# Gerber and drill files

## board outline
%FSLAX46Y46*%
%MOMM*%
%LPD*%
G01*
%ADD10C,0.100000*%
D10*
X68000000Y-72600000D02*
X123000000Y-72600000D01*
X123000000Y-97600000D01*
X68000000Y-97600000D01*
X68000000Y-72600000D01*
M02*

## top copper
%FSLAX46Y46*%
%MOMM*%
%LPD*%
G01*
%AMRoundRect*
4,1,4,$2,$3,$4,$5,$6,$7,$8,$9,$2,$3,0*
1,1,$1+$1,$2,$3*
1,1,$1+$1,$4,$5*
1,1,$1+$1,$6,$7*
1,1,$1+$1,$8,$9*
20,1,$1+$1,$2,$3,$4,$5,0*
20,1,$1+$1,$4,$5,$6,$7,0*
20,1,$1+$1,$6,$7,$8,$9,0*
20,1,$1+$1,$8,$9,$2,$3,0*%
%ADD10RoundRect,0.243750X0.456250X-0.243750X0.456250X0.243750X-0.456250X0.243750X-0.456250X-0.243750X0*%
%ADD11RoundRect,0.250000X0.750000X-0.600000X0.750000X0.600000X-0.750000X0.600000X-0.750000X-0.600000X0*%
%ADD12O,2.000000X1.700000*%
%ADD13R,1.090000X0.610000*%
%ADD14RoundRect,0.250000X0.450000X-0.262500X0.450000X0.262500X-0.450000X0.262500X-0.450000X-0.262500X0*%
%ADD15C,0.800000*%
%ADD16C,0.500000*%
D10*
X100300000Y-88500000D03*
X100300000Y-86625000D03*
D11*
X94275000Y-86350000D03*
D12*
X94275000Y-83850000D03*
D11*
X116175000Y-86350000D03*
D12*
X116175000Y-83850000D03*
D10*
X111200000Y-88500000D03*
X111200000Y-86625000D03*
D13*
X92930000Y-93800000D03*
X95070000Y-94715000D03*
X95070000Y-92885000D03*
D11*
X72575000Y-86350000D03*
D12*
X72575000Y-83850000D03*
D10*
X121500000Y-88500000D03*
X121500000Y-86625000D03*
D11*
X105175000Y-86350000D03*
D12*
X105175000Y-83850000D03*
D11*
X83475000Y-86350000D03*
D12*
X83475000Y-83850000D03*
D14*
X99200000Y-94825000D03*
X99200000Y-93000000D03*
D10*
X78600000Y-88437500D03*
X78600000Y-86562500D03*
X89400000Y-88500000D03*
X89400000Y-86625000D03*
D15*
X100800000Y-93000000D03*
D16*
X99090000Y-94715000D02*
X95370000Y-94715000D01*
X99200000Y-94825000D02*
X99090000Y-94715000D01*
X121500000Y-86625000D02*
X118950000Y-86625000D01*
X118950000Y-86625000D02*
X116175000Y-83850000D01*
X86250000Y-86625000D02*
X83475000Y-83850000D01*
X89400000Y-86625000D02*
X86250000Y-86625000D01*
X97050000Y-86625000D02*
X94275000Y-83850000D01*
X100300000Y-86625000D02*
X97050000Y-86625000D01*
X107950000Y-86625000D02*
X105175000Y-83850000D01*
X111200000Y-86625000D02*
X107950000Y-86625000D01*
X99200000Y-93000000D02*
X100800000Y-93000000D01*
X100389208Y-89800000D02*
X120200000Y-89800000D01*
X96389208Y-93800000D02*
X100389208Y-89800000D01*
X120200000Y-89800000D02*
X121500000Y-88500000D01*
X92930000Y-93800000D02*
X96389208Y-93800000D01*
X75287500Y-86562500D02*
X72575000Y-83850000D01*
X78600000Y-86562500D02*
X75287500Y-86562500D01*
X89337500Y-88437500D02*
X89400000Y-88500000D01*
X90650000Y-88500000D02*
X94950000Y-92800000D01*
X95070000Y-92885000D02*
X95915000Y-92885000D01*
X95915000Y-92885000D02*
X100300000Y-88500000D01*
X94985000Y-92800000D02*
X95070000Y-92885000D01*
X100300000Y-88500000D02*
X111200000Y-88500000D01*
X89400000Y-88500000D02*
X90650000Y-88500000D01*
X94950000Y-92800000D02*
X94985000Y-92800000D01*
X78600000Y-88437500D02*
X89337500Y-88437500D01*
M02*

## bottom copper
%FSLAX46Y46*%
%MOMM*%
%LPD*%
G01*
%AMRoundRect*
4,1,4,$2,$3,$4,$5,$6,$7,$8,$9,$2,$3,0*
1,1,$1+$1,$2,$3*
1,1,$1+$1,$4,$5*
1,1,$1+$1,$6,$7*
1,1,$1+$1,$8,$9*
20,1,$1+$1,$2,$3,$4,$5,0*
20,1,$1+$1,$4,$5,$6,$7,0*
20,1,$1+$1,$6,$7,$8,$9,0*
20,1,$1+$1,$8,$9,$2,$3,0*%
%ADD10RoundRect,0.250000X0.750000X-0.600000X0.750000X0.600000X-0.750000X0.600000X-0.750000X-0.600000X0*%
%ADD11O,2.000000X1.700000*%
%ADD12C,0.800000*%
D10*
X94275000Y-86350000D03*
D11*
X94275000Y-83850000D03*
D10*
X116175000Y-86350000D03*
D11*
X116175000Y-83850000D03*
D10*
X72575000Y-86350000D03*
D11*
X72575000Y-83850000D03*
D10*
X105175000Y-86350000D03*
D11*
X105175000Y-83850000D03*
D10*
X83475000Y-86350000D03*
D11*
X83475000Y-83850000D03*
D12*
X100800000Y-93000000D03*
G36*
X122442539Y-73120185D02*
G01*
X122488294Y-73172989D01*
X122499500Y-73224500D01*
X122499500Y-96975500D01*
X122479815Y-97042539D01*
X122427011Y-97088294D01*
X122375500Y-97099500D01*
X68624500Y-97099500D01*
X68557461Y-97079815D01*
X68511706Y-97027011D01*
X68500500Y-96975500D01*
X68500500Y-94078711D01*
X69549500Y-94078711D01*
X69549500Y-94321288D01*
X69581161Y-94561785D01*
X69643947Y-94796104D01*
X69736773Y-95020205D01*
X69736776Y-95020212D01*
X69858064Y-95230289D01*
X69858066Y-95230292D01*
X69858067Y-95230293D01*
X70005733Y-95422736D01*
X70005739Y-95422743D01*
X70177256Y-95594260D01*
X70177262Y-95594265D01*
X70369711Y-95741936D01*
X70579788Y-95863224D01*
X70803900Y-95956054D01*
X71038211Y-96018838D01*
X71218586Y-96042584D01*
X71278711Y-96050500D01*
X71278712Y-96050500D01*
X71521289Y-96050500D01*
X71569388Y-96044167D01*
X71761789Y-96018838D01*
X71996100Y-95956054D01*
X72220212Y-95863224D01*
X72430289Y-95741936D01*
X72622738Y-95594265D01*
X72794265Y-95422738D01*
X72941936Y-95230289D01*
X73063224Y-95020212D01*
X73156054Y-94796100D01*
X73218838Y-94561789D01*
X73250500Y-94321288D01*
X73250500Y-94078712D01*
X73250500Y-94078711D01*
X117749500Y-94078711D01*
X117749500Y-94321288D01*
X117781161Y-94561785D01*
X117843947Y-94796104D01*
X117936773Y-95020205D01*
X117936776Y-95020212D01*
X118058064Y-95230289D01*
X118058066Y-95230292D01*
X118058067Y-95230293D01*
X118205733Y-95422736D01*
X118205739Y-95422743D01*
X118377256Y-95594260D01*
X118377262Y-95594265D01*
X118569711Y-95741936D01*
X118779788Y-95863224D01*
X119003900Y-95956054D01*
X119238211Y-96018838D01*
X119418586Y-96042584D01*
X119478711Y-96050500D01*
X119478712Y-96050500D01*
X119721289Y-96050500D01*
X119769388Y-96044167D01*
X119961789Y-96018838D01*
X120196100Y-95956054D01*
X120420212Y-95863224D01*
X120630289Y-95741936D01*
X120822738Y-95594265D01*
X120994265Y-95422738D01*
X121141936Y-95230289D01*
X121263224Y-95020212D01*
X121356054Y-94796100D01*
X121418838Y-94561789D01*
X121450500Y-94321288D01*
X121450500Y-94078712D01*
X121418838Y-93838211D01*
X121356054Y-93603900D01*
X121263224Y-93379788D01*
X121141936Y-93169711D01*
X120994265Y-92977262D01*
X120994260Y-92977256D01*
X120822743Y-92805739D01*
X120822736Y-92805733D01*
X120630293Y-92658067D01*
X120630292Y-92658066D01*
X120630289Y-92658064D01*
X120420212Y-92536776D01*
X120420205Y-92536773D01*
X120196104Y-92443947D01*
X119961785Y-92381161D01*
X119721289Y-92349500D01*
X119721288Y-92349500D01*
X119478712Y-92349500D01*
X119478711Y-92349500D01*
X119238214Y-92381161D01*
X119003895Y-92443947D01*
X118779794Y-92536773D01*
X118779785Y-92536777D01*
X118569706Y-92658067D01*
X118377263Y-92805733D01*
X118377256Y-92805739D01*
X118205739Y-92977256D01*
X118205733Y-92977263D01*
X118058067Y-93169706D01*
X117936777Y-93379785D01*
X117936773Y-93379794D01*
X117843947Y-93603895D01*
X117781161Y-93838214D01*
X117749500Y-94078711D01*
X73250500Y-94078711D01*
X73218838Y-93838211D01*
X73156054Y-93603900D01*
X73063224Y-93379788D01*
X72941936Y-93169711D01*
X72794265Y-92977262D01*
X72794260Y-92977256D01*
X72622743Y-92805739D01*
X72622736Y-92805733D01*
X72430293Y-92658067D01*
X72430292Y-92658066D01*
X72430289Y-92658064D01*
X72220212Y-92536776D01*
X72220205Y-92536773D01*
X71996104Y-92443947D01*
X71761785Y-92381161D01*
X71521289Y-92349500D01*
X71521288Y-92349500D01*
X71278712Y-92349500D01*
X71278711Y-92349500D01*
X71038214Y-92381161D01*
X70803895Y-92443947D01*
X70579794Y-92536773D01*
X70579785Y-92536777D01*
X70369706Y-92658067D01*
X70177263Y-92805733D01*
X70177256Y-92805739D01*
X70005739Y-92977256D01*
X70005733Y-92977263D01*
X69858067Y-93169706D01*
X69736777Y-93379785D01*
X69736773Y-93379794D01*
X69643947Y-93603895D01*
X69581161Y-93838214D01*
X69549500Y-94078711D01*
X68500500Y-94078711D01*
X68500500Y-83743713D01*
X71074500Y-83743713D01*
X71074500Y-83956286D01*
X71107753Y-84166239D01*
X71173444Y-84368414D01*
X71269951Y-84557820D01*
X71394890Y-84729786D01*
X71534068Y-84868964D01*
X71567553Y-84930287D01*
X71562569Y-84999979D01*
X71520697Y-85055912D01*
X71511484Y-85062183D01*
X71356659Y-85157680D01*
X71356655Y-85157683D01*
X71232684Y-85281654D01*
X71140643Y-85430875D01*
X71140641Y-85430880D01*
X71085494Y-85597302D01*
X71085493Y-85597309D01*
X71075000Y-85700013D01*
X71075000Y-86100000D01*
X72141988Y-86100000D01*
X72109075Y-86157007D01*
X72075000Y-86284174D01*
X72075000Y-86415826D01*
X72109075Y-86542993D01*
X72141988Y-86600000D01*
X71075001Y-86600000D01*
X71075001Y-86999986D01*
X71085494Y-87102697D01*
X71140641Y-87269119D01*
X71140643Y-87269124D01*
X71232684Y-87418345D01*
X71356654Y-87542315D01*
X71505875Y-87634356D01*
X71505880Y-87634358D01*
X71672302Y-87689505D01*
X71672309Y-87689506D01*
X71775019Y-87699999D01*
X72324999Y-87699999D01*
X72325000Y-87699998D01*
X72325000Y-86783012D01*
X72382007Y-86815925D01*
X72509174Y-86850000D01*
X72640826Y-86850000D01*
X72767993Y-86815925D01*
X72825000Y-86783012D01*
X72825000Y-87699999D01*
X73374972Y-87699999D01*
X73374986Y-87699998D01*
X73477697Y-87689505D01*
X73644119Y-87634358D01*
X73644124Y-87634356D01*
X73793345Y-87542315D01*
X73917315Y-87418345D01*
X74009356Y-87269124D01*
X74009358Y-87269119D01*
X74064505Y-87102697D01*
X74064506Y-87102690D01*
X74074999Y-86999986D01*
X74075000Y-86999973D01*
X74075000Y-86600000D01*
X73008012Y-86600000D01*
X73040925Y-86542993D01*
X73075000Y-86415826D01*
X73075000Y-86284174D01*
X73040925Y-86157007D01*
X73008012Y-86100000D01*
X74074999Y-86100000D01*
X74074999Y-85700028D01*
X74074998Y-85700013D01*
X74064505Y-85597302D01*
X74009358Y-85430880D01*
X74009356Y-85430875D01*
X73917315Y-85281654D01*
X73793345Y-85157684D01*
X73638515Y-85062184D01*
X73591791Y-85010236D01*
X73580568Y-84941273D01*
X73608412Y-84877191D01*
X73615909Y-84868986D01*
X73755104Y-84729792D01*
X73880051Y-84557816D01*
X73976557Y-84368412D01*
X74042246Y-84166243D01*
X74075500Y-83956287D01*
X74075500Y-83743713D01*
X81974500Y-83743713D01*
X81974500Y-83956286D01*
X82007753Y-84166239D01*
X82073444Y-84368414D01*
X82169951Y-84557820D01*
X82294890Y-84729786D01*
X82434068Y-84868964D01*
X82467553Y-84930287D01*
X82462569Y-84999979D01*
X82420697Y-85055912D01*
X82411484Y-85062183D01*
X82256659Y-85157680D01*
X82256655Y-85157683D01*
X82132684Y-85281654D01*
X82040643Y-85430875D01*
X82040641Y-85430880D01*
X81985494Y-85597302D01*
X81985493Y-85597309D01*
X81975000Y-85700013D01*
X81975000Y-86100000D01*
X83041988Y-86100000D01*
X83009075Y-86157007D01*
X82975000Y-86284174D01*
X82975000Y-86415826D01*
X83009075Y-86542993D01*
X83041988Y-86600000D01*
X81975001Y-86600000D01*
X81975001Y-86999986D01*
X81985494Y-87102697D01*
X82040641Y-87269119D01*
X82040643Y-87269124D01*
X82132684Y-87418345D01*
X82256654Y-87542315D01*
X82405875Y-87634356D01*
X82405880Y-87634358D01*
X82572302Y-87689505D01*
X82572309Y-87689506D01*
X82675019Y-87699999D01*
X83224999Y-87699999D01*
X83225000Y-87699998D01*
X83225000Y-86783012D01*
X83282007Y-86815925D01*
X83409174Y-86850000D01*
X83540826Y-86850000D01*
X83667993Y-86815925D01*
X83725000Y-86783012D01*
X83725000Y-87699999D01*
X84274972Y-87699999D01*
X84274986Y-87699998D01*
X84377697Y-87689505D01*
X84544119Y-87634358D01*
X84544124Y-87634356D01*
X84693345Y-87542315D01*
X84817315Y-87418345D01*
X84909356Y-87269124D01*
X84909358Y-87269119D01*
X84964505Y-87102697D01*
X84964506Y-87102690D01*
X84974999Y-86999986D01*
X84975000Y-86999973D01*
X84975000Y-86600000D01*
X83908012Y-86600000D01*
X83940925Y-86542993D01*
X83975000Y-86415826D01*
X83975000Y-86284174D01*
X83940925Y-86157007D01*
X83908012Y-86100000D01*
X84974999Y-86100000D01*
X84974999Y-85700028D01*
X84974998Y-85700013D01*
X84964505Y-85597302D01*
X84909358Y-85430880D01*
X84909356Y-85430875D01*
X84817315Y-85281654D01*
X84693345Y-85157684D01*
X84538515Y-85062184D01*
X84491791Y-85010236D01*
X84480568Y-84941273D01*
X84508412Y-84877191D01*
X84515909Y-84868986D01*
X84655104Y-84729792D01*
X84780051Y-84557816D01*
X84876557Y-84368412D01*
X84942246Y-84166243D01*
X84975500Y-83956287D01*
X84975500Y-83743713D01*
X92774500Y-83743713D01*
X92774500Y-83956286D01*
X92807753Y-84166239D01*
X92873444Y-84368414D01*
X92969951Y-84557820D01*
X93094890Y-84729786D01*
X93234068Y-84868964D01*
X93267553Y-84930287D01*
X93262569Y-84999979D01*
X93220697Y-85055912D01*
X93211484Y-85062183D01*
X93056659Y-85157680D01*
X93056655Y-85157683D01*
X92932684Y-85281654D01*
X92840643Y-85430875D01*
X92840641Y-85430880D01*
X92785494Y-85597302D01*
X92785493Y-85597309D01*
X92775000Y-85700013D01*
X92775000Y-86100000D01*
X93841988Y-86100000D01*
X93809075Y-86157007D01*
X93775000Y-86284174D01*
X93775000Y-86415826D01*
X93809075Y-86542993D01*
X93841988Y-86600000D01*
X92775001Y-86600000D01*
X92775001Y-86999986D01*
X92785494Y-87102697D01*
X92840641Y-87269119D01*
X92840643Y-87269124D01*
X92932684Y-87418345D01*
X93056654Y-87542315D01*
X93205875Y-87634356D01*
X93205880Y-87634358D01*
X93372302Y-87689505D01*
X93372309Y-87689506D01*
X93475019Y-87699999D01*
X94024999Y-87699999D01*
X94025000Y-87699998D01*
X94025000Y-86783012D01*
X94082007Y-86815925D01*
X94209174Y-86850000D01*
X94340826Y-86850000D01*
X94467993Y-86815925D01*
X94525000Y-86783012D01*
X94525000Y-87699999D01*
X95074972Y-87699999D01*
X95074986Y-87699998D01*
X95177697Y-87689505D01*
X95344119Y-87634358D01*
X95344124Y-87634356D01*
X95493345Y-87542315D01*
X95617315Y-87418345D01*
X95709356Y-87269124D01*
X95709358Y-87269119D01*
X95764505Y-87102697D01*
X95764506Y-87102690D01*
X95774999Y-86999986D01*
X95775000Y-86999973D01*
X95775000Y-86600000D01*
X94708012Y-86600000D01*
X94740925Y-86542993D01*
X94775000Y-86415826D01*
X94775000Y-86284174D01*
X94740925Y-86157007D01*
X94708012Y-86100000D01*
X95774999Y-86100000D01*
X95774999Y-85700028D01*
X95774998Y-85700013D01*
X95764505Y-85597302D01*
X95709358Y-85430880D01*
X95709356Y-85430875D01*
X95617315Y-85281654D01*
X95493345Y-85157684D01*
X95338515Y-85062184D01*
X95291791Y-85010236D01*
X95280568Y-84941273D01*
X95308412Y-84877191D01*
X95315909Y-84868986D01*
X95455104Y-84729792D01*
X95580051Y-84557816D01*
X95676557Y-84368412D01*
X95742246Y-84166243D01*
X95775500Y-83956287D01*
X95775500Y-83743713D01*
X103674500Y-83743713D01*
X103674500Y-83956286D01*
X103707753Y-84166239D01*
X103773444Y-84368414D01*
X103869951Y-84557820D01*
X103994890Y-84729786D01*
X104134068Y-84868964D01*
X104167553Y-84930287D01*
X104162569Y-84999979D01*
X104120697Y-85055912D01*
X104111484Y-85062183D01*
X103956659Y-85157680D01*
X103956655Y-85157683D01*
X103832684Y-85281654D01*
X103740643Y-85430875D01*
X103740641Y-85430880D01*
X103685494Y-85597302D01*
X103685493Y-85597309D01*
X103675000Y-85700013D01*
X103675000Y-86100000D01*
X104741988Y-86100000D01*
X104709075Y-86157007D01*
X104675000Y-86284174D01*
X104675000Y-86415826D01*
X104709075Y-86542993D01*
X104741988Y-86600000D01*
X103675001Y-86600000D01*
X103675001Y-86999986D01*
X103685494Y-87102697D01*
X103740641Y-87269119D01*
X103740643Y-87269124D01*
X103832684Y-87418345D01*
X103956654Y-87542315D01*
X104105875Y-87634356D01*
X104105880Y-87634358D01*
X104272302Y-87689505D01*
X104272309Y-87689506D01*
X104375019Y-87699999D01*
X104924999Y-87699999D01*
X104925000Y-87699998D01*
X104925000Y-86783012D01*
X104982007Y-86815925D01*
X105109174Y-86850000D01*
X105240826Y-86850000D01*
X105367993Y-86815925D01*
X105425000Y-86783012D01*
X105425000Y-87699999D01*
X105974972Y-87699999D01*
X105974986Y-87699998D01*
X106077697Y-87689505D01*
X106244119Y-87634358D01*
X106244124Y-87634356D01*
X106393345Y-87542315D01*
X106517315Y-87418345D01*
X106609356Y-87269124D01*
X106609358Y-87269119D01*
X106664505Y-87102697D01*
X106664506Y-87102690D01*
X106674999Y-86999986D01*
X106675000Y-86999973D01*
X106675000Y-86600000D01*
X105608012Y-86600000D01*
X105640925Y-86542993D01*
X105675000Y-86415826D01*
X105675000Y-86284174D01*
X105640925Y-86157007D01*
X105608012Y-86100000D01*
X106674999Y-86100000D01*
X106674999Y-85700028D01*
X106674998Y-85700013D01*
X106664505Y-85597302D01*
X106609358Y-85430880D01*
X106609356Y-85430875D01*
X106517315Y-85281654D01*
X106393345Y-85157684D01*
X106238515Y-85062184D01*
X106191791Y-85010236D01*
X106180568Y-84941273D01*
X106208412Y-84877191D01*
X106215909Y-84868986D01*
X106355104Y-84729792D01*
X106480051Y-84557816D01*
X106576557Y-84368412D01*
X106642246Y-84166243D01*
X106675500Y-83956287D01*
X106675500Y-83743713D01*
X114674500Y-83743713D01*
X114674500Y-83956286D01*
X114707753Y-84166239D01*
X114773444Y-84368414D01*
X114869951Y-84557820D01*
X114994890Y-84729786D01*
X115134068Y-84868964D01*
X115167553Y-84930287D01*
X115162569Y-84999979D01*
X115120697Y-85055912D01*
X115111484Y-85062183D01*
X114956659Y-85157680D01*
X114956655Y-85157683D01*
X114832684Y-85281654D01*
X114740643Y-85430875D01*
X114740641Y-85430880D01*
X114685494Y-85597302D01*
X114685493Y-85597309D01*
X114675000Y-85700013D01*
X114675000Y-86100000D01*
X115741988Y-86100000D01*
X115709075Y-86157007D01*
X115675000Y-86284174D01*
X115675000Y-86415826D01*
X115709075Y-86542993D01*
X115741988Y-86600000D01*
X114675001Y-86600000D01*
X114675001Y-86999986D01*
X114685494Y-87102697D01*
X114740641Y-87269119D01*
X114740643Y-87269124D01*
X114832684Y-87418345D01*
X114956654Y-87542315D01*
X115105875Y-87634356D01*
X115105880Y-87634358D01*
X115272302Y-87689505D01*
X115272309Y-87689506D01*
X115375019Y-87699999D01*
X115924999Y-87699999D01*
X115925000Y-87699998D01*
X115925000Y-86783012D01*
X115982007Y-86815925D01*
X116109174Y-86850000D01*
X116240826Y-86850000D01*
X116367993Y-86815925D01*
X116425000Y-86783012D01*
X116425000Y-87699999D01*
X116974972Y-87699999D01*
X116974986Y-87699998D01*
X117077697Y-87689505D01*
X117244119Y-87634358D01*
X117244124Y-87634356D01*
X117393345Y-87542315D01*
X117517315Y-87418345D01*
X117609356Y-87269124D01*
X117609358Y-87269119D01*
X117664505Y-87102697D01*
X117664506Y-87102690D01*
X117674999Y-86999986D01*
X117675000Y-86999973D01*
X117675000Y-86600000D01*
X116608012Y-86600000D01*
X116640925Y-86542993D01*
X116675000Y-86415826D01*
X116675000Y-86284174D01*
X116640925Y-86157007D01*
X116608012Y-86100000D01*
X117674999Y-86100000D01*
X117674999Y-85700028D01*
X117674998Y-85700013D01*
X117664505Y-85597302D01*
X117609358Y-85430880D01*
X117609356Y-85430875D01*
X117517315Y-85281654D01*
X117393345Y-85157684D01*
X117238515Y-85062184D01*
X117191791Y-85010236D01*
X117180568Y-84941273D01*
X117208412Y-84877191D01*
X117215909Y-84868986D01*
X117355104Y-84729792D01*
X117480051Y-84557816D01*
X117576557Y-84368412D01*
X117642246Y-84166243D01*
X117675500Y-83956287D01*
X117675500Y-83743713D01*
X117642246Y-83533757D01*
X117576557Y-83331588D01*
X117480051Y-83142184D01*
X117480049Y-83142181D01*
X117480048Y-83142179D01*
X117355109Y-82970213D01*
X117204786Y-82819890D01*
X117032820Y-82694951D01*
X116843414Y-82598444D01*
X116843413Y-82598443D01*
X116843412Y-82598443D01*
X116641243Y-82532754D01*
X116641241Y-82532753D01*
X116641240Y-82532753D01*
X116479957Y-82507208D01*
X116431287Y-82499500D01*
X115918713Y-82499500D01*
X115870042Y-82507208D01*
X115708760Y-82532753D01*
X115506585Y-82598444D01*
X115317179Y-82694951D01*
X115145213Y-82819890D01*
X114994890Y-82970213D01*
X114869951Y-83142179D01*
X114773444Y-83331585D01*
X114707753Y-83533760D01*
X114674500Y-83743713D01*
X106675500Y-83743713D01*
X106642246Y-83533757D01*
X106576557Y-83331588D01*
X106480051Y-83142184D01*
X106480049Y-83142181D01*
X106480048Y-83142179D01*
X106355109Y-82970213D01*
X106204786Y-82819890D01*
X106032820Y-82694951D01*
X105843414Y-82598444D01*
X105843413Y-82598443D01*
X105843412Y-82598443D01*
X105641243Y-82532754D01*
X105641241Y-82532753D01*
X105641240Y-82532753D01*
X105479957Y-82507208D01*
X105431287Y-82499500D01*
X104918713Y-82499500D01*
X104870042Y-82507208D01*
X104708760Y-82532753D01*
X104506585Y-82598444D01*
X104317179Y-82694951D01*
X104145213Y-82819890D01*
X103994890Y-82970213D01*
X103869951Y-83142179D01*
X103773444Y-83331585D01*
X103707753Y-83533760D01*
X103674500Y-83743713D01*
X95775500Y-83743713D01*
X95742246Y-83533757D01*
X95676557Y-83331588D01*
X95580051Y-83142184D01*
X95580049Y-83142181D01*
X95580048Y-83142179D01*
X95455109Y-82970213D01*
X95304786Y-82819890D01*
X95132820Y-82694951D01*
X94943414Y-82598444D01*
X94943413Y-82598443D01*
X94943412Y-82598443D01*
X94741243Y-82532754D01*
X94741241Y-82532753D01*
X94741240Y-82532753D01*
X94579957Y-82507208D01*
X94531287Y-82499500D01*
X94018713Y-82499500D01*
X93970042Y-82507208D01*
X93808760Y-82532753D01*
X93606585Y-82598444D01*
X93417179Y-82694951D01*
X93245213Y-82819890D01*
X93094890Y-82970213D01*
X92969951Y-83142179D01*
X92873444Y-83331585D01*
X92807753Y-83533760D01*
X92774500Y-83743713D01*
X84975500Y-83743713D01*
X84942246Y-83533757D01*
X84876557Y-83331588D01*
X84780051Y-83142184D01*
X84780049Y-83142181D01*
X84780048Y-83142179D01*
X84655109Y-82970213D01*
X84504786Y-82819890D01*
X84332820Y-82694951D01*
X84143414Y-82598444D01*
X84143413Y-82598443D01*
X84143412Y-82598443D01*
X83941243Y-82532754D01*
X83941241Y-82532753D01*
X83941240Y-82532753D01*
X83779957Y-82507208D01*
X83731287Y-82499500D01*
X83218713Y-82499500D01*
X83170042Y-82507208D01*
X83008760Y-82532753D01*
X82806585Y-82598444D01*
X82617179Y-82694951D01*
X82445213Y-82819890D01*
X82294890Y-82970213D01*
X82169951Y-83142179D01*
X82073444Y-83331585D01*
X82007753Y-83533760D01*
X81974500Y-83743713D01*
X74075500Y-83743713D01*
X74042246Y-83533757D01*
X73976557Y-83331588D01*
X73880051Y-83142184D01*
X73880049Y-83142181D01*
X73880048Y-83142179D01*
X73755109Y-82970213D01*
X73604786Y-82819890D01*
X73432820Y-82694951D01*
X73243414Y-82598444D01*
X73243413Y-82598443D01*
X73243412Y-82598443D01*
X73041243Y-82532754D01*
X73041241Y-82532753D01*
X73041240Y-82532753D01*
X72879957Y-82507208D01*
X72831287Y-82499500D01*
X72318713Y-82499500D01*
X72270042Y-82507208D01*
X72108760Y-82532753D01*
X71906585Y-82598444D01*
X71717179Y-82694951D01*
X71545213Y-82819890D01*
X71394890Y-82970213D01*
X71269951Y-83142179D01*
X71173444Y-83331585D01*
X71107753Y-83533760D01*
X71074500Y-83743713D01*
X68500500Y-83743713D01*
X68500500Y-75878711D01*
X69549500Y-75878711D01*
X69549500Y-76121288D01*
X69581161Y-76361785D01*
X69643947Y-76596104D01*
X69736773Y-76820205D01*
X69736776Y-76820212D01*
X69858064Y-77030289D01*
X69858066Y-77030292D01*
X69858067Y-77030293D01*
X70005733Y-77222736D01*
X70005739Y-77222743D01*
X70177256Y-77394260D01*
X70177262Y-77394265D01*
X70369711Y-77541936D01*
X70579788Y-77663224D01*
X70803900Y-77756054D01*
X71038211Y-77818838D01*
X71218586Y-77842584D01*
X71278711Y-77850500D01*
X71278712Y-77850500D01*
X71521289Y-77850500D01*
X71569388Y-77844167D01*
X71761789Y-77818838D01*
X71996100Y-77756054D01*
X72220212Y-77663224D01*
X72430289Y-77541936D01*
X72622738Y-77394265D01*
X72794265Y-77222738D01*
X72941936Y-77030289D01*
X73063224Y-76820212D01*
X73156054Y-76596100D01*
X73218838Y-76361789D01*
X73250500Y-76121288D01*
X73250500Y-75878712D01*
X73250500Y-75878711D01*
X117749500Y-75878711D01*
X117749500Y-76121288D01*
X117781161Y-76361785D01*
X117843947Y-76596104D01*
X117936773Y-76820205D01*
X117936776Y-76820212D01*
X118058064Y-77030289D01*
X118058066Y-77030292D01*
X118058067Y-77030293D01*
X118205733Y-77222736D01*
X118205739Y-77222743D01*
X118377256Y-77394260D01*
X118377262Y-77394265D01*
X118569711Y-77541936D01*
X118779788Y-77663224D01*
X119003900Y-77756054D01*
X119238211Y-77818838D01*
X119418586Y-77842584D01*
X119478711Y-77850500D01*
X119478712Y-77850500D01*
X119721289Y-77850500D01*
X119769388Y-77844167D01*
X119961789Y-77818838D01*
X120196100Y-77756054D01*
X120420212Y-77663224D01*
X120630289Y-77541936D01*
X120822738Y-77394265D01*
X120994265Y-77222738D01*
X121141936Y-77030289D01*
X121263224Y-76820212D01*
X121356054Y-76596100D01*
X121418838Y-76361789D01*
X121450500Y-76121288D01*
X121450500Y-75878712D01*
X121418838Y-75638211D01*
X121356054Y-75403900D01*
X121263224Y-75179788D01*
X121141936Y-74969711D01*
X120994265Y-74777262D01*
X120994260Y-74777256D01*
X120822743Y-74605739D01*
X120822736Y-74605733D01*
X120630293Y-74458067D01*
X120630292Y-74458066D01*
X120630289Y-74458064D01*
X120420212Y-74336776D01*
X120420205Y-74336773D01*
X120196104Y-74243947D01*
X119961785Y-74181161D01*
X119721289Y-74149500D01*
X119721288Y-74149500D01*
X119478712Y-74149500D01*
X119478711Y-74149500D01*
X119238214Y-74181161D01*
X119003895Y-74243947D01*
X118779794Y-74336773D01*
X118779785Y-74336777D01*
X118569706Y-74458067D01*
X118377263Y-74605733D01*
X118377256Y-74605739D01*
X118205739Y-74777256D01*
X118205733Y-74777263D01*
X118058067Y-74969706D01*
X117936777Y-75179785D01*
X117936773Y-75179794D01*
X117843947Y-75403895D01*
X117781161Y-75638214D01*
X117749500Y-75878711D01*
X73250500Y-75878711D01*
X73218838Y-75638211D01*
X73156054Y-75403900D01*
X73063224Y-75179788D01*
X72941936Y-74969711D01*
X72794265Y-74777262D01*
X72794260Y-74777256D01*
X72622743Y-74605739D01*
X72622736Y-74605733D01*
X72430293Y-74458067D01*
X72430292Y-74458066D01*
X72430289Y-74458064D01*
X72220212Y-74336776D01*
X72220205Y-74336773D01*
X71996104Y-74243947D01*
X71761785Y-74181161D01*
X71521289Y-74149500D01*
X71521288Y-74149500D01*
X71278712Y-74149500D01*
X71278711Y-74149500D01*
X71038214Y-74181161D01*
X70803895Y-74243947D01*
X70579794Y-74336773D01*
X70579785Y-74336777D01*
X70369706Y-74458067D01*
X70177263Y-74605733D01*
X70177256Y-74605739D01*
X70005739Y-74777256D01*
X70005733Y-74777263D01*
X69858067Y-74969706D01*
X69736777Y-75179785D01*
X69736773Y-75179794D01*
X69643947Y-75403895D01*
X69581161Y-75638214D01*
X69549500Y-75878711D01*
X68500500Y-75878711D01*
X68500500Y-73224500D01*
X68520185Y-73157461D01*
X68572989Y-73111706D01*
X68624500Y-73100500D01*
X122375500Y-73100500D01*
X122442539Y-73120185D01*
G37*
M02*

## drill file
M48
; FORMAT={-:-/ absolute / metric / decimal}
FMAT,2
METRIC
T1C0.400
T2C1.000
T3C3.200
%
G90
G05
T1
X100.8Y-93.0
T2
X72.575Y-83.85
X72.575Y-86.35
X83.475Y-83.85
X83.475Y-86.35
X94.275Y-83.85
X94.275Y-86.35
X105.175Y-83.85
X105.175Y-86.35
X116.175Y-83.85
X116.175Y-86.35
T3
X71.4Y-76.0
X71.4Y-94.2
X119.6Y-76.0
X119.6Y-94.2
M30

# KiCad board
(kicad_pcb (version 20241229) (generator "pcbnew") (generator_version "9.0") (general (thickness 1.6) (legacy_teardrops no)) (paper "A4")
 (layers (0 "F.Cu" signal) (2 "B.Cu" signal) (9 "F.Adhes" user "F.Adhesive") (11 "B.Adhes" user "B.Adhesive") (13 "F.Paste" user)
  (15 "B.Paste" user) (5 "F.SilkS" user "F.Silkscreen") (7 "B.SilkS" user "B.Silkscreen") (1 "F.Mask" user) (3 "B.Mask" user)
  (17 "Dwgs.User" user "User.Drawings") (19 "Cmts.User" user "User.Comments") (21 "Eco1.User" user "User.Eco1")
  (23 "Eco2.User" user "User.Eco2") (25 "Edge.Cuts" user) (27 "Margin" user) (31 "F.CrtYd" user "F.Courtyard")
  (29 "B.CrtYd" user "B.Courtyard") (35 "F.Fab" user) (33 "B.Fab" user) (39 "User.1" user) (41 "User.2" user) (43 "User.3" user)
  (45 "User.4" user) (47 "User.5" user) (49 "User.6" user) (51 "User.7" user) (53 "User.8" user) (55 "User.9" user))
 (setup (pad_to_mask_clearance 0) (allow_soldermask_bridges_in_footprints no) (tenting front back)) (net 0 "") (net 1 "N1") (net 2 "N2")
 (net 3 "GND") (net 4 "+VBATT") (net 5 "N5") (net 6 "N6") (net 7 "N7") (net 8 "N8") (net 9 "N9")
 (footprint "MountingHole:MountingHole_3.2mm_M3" (layer "F.Cu") (at 119.6 94.2 90)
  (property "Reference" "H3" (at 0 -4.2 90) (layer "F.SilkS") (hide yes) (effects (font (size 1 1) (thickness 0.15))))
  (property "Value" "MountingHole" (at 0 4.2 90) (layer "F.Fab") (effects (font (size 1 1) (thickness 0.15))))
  (pad "" np_thru_hole circle (at 0 0 90) (size 3.2 3.2) (drill 3.2) (layers "*.Cu" "*.Mask")))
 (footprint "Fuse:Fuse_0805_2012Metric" (layer "F.Cu") (at 100.3 87.5625 90)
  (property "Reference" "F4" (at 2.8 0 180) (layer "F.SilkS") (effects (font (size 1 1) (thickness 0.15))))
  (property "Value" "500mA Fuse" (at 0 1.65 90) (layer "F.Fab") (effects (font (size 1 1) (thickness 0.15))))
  (pad "1" smd roundrect (at -0.9375 0 90) (size 0.975 1.4) (layers "F.Cu" "F.Mask" "F.Paste") (roundrect_rratio 0.25) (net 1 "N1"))
  (pad "2" smd roundrect (at 0.9375 0 90) (size 0.975 1.4) (layers "F.Cu" "F.Mask" "F.Paste") (roundrect_rratio 0.25) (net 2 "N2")))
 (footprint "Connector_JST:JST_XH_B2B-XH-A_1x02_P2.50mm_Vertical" (layer "F.Cu") (at 94.275 86.35 90)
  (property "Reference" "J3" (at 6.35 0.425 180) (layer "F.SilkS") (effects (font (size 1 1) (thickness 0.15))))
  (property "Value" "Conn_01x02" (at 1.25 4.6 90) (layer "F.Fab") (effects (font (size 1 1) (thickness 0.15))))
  (pad "1" thru_hole roundrect (at 0 0 90) (size 1.7 2) (drill 1) (layers "*.Cu" "*.Mask") (remove_unused_layers no)
   (roundrect_rratio 0.147059) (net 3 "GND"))
  (pad "2" thru_hole oval (at 2.5 0 90) (size 1.7 2) (drill 1) (layers "*.Cu" "*.Mask") (remove_unused_layers no) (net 2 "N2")))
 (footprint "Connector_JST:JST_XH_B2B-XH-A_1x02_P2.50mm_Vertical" (layer "F.Cu") (at 116.175 86.35 90)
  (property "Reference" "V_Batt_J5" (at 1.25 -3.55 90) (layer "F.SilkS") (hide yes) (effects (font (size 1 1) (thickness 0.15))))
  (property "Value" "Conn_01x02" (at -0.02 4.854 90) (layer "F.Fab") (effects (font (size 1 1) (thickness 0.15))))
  (pad "1" thru_hole roundrect (at 0 0 90) (size 1.7 2) (drill 1) (layers "*.Cu" "*.Mask") (remove_unused_layers no)
   (roundrect_rratio 0.147059) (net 3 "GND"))
  (pad "2" thru_hole oval (at 2.5 0 90) (size 1.7 2) (drill 1) (layers "*.Cu" "*.Mask") (remove_unused_layers no) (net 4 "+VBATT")))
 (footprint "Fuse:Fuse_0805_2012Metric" (layer "F.Cu") (at 111.2 87.5625 90)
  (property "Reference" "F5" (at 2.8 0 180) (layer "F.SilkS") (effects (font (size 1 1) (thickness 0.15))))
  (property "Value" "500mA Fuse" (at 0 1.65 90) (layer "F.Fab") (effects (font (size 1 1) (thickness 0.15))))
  (pad "1" smd roundrect (at -0.9375 0 90) (size 0.975 1.4) (layers "F.Cu" "F.Mask" "F.Paste") (roundrect_rratio 0.25) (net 1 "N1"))
  (pad "2" smd roundrect (at 0.9375 0 90) (size 0.975 1.4) (layers "F.Cu" "F.Mask" "F.Paste") (roundrect_rratio 0.25) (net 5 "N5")))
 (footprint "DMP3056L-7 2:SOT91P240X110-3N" (layer "F.Cu") (at 94 93.8 180)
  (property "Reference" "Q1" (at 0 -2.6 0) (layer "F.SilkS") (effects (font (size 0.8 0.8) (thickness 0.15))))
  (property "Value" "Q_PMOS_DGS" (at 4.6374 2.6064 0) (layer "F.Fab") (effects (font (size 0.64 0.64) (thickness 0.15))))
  (pad "1" smd rect (at 1.07 0 180) (size 1.09 0.61) (layers "F.Cu" "F.Mask" "F.Paste") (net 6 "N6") (solder_mask_margin 0.102))
  (pad "2" smd rect (at -1.07 -0.915 180) (size 1.09 0.61) (layers "F.Cu" "F.Mask" "F.Paste") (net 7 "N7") (solder_mask_margin 0.102))
  (pad "3" smd rect (at -1.07 0.915 180) (size 1.09 0.61) (layers "F.Cu" "F.Mask" "F.Paste") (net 1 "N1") (solder_mask_margin 0.102)))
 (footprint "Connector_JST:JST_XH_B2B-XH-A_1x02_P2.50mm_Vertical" (layer "F.Cu") (at 72.575 86.35 90)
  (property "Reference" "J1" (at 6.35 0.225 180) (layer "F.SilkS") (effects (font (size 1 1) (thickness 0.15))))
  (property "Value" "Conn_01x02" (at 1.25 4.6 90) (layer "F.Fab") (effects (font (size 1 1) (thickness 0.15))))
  (pad "1" thru_hole roundrect (at 0 0 90) (size 1.7 2) (drill 1) (layers "*.Cu" "*.Mask") (remove_unused_layers no)
   (roundrect_rratio 0.147059) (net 3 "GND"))
  (pad "2" thru_hole oval (at 2.5 0 90) (size 1.7 2) (drill 1) (layers "*.Cu" "*.Mask") (remove_unused_layers no) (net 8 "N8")))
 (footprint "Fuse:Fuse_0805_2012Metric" (layer "F.Cu") (at 121.5 87.5625 90)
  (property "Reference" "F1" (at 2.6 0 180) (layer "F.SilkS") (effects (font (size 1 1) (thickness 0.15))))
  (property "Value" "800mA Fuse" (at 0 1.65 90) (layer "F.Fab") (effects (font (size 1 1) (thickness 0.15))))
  (pad "1" smd roundrect (at -0.9375 0 90) (size 0.975 1.4) (layers "F.Cu" "F.Mask" "F.Paste") (roundrect_rratio 0.25) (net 6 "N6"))
  (pad "2" smd roundrect (at 0.9375 0 90) (size 0.975 1.4) (layers "F.Cu" "F.Mask" "F.Paste") (roundrect_rratio 0.25) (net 4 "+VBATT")))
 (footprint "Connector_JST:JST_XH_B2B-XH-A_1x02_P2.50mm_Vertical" (layer "F.Cu") (at 105.175 86.35 90)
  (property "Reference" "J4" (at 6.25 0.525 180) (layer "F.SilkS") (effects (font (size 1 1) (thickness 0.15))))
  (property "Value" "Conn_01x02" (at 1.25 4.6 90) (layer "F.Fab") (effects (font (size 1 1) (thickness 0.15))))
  (pad "1" thru_hole roundrect (at 0 0 90) (size 1.7 2) (drill 1) (layers "*.Cu" "*.Mask") (remove_unused_layers no)
   (roundrect_rratio 0.147059) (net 3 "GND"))
  (pad "2" thru_hole oval (at 2.5 0 90) (size 1.7 2) (drill 1) (layers "*.Cu" "*.Mask") (remove_unused_layers no) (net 5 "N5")))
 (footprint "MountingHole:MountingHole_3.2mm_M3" (layer "F.Cu") (at 71.4 94.2 90)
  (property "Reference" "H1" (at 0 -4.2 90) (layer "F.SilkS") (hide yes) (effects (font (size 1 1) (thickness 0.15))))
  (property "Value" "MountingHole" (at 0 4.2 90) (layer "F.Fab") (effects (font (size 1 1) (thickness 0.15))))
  (pad "" np_thru_hole circle (at 0 0 90) (size 3.2 3.2) (drill 3.2) (layers "*.Cu" "*.Mask")))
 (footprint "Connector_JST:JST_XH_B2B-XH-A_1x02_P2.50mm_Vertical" (layer "F.Cu") (at 83.475 86.35 90)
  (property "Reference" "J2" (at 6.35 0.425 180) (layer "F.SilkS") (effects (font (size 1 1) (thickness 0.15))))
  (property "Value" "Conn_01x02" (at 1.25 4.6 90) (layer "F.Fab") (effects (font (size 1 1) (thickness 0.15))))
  (pad "1" thru_hole roundrect (at 0 0 90) (size 1.7 2) (drill 1) (layers "*.Cu" "*.Mask") (remove_unused_layers no)
   (roundrect_rratio 0.147059) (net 3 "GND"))
  (pad "2" thru_hole oval (at 2.5 0 90) (size 1.7 2) (drill 1) (layers "*.Cu" "*.Mask") (remove_unused_layers no) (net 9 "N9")))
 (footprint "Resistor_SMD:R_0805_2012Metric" (layer "F.Cu") (at 99.2 93.9125 90)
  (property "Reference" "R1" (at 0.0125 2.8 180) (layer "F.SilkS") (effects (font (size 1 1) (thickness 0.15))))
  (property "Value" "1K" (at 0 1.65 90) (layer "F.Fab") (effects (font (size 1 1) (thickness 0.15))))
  (pad "1" smd roundrect (at -0.9125 0 90) (size 1.025 1.4) (layers "F.Cu" "F.Mask" "F.Paste") (roundrect_rratio 0.243902) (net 7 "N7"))
  (pad "2" smd roundrect (at 0.9125 0 90) (size 1.025 1.4) (layers "F.Cu" "F.Mask" "F.Paste") (roundrect_rratio 0.243902) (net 3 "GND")))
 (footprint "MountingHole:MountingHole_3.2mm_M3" (layer "F.Cu") (at 119.6 76 90)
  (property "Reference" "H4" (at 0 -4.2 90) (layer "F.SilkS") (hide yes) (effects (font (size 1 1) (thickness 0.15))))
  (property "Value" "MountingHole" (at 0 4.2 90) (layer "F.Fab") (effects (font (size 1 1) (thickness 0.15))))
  (pad "" np_thru_hole circle (at 0 0 90) (size 3.2 3.2) (drill 3.2) (layers "*.Cu" "*.Mask")))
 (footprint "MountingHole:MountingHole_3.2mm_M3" (layer "F.Cu") (at 71.4 76 90)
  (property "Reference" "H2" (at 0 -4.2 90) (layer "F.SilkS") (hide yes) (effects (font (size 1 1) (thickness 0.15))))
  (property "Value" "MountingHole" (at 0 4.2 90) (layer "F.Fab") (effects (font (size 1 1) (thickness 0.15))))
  (pad "" np_thru_hole circle (at 0 0 90) (size 3.2 3.2) (drill 3.2) (layers "*.Cu" "*.Mask")))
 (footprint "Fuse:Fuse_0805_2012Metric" (layer "F.Cu") (at 78.6 87.5 90)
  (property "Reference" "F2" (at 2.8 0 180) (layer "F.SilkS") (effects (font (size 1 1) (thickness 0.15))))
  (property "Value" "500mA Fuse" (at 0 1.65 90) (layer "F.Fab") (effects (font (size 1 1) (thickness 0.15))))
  (pad "1" smd roundrect (at -0.9375 0 90) (size 0.975 1.4) (layers "F.Cu" "F.Mask" "F.Paste") (roundrect_rratio 0.25) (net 1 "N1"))
  (pad "2" smd roundrect (at 0.9375 0 90) (size 0.975 1.4) (layers "F.Cu" "F.Mask" "F.Paste") (roundrect_rratio 0.25) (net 8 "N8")))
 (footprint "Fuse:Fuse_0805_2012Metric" (layer "F.Cu") (at 89.4 87.5625 90)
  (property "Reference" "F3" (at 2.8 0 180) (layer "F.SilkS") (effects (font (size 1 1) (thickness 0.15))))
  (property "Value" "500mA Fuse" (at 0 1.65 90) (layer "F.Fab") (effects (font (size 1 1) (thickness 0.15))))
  (pad "1" smd roundrect (at -0.9375 0 90) (size 0.975 1.4) (layers "F.Cu" "F.Mask" "F.Paste") (roundrect_rratio 0.25) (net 1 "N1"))
  (pad "2" smd roundrect (at 0.9375 0 90) (size 0.975 1.4) (layers "F.Cu" "F.Mask" "F.Paste") (roundrect_rratio 0.25) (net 9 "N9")))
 (gr_rect (start 68 72.6) (end 123 97.6) (stroke (width 0.1) (type solid)) (fill no) (layer "Edge.Cuts"))
 (segment (start 99.09 94.715) (end 95.37 94.715) (width 0.5) (layer "F.Cu") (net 7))
 (segment (start 99.2 94.825) (end 99.09 94.715) (width 0.5) (layer "F.Cu") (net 7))
 (segment (start 121.5 86.625) (end 118.95 86.625) (width 0.5) (layer "F.Cu") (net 4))
 (segment (start 118.95 86.625) (end 116.175 83.85) (width 0.5) (layer "F.Cu") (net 4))
 (segment (start 86.25 86.625) (end 83.475 83.85) (width 0.5) (layer "F.Cu") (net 9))
 (segment (start 89.4 86.625) (end 86.25 86.625) (width 0.5) (layer "F.Cu") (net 9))
 (segment (start 97.05 86.625) (end 94.275 83.85) (width 0.5) (layer "F.Cu") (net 2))
 (segment (start 100.3 86.625) (end 97.05 86.625) (width 0.5) (layer "F.Cu") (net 2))
 (segment (start 107.95 86.625) (end 105.175 83.85) (width 0.5) (layer "F.Cu") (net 5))
 (segment (start 111.2 86.625) (end 107.95 86.625) (width 0.5) (layer "F.Cu") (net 5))
 (segment (start 99.2 93) (end 100.8 93) (width 0.5) (layer "F.Cu") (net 3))
 (via (at 100.8 93) (size 0.8) (drill 0.4) (layers "F.Cu" "B.Cu") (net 3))
 (segment (start 100.389208 89.8) (end 120.2 89.8) (width 0.5) (layer "F.Cu") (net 6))
 (segment (start 96.389208 93.8) (end 100.389208 89.8) (width 0.5) (layer "F.Cu") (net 6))
 (segment (start 120.2 89.8) (end 121.5 88.5) (width 0.5) (layer "F.Cu") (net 6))
 (segment (start 92.93 93.8) (end 96.389208 93.8) (width 0.5) (layer "F.Cu") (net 6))
 (segment (start 75.2875 86.5625) (end 72.575 83.85) (width 0.5) (layer "F.Cu") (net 8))
 (segment (start 78.6 86.5625) (end 75.2875 86.5625) (width 0.5) (layer "F.Cu") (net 8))
 (segment (start 89.3375 88.4375) (end 89.4 88.5) (width 0.5) (layer "F.Cu") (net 1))
 (segment (start 90.65 88.5) (end 94.95 92.8) (width 0.5) (layer "F.Cu") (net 1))
 (segment (start 95.07 92.885) (end 95.915 92.885) (width 0.5) (layer "F.Cu") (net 1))
 (segment (start 95.915 92.885) (end 100.3 88.5) (width 0.5) (layer "F.Cu") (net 1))
 (segment (start 94.985 92.8) (end 95.07 92.885) (width 0.5) (layer "F.Cu") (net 1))
 (segment (start 100.3 88.5) (end 111.2 88.5) (width 0.5) (layer "F.Cu") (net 1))
 (segment (start 89.4 88.5) (end 90.65 88.5) (width 0.5) (layer "F.Cu") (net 1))
 (segment (start 94.95 92.8) (end 94.985 92.8) (width 0.5) (layer "F.Cu") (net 1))
 (segment (start 78.6 88.4375) (end 89.3375 88.4375) (width 0.5) (layer "F.Cu") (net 1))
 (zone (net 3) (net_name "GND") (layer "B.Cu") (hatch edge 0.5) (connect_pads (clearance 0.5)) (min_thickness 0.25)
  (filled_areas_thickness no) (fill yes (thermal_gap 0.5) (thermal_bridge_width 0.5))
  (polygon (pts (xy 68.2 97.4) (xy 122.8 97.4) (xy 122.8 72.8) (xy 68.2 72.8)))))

